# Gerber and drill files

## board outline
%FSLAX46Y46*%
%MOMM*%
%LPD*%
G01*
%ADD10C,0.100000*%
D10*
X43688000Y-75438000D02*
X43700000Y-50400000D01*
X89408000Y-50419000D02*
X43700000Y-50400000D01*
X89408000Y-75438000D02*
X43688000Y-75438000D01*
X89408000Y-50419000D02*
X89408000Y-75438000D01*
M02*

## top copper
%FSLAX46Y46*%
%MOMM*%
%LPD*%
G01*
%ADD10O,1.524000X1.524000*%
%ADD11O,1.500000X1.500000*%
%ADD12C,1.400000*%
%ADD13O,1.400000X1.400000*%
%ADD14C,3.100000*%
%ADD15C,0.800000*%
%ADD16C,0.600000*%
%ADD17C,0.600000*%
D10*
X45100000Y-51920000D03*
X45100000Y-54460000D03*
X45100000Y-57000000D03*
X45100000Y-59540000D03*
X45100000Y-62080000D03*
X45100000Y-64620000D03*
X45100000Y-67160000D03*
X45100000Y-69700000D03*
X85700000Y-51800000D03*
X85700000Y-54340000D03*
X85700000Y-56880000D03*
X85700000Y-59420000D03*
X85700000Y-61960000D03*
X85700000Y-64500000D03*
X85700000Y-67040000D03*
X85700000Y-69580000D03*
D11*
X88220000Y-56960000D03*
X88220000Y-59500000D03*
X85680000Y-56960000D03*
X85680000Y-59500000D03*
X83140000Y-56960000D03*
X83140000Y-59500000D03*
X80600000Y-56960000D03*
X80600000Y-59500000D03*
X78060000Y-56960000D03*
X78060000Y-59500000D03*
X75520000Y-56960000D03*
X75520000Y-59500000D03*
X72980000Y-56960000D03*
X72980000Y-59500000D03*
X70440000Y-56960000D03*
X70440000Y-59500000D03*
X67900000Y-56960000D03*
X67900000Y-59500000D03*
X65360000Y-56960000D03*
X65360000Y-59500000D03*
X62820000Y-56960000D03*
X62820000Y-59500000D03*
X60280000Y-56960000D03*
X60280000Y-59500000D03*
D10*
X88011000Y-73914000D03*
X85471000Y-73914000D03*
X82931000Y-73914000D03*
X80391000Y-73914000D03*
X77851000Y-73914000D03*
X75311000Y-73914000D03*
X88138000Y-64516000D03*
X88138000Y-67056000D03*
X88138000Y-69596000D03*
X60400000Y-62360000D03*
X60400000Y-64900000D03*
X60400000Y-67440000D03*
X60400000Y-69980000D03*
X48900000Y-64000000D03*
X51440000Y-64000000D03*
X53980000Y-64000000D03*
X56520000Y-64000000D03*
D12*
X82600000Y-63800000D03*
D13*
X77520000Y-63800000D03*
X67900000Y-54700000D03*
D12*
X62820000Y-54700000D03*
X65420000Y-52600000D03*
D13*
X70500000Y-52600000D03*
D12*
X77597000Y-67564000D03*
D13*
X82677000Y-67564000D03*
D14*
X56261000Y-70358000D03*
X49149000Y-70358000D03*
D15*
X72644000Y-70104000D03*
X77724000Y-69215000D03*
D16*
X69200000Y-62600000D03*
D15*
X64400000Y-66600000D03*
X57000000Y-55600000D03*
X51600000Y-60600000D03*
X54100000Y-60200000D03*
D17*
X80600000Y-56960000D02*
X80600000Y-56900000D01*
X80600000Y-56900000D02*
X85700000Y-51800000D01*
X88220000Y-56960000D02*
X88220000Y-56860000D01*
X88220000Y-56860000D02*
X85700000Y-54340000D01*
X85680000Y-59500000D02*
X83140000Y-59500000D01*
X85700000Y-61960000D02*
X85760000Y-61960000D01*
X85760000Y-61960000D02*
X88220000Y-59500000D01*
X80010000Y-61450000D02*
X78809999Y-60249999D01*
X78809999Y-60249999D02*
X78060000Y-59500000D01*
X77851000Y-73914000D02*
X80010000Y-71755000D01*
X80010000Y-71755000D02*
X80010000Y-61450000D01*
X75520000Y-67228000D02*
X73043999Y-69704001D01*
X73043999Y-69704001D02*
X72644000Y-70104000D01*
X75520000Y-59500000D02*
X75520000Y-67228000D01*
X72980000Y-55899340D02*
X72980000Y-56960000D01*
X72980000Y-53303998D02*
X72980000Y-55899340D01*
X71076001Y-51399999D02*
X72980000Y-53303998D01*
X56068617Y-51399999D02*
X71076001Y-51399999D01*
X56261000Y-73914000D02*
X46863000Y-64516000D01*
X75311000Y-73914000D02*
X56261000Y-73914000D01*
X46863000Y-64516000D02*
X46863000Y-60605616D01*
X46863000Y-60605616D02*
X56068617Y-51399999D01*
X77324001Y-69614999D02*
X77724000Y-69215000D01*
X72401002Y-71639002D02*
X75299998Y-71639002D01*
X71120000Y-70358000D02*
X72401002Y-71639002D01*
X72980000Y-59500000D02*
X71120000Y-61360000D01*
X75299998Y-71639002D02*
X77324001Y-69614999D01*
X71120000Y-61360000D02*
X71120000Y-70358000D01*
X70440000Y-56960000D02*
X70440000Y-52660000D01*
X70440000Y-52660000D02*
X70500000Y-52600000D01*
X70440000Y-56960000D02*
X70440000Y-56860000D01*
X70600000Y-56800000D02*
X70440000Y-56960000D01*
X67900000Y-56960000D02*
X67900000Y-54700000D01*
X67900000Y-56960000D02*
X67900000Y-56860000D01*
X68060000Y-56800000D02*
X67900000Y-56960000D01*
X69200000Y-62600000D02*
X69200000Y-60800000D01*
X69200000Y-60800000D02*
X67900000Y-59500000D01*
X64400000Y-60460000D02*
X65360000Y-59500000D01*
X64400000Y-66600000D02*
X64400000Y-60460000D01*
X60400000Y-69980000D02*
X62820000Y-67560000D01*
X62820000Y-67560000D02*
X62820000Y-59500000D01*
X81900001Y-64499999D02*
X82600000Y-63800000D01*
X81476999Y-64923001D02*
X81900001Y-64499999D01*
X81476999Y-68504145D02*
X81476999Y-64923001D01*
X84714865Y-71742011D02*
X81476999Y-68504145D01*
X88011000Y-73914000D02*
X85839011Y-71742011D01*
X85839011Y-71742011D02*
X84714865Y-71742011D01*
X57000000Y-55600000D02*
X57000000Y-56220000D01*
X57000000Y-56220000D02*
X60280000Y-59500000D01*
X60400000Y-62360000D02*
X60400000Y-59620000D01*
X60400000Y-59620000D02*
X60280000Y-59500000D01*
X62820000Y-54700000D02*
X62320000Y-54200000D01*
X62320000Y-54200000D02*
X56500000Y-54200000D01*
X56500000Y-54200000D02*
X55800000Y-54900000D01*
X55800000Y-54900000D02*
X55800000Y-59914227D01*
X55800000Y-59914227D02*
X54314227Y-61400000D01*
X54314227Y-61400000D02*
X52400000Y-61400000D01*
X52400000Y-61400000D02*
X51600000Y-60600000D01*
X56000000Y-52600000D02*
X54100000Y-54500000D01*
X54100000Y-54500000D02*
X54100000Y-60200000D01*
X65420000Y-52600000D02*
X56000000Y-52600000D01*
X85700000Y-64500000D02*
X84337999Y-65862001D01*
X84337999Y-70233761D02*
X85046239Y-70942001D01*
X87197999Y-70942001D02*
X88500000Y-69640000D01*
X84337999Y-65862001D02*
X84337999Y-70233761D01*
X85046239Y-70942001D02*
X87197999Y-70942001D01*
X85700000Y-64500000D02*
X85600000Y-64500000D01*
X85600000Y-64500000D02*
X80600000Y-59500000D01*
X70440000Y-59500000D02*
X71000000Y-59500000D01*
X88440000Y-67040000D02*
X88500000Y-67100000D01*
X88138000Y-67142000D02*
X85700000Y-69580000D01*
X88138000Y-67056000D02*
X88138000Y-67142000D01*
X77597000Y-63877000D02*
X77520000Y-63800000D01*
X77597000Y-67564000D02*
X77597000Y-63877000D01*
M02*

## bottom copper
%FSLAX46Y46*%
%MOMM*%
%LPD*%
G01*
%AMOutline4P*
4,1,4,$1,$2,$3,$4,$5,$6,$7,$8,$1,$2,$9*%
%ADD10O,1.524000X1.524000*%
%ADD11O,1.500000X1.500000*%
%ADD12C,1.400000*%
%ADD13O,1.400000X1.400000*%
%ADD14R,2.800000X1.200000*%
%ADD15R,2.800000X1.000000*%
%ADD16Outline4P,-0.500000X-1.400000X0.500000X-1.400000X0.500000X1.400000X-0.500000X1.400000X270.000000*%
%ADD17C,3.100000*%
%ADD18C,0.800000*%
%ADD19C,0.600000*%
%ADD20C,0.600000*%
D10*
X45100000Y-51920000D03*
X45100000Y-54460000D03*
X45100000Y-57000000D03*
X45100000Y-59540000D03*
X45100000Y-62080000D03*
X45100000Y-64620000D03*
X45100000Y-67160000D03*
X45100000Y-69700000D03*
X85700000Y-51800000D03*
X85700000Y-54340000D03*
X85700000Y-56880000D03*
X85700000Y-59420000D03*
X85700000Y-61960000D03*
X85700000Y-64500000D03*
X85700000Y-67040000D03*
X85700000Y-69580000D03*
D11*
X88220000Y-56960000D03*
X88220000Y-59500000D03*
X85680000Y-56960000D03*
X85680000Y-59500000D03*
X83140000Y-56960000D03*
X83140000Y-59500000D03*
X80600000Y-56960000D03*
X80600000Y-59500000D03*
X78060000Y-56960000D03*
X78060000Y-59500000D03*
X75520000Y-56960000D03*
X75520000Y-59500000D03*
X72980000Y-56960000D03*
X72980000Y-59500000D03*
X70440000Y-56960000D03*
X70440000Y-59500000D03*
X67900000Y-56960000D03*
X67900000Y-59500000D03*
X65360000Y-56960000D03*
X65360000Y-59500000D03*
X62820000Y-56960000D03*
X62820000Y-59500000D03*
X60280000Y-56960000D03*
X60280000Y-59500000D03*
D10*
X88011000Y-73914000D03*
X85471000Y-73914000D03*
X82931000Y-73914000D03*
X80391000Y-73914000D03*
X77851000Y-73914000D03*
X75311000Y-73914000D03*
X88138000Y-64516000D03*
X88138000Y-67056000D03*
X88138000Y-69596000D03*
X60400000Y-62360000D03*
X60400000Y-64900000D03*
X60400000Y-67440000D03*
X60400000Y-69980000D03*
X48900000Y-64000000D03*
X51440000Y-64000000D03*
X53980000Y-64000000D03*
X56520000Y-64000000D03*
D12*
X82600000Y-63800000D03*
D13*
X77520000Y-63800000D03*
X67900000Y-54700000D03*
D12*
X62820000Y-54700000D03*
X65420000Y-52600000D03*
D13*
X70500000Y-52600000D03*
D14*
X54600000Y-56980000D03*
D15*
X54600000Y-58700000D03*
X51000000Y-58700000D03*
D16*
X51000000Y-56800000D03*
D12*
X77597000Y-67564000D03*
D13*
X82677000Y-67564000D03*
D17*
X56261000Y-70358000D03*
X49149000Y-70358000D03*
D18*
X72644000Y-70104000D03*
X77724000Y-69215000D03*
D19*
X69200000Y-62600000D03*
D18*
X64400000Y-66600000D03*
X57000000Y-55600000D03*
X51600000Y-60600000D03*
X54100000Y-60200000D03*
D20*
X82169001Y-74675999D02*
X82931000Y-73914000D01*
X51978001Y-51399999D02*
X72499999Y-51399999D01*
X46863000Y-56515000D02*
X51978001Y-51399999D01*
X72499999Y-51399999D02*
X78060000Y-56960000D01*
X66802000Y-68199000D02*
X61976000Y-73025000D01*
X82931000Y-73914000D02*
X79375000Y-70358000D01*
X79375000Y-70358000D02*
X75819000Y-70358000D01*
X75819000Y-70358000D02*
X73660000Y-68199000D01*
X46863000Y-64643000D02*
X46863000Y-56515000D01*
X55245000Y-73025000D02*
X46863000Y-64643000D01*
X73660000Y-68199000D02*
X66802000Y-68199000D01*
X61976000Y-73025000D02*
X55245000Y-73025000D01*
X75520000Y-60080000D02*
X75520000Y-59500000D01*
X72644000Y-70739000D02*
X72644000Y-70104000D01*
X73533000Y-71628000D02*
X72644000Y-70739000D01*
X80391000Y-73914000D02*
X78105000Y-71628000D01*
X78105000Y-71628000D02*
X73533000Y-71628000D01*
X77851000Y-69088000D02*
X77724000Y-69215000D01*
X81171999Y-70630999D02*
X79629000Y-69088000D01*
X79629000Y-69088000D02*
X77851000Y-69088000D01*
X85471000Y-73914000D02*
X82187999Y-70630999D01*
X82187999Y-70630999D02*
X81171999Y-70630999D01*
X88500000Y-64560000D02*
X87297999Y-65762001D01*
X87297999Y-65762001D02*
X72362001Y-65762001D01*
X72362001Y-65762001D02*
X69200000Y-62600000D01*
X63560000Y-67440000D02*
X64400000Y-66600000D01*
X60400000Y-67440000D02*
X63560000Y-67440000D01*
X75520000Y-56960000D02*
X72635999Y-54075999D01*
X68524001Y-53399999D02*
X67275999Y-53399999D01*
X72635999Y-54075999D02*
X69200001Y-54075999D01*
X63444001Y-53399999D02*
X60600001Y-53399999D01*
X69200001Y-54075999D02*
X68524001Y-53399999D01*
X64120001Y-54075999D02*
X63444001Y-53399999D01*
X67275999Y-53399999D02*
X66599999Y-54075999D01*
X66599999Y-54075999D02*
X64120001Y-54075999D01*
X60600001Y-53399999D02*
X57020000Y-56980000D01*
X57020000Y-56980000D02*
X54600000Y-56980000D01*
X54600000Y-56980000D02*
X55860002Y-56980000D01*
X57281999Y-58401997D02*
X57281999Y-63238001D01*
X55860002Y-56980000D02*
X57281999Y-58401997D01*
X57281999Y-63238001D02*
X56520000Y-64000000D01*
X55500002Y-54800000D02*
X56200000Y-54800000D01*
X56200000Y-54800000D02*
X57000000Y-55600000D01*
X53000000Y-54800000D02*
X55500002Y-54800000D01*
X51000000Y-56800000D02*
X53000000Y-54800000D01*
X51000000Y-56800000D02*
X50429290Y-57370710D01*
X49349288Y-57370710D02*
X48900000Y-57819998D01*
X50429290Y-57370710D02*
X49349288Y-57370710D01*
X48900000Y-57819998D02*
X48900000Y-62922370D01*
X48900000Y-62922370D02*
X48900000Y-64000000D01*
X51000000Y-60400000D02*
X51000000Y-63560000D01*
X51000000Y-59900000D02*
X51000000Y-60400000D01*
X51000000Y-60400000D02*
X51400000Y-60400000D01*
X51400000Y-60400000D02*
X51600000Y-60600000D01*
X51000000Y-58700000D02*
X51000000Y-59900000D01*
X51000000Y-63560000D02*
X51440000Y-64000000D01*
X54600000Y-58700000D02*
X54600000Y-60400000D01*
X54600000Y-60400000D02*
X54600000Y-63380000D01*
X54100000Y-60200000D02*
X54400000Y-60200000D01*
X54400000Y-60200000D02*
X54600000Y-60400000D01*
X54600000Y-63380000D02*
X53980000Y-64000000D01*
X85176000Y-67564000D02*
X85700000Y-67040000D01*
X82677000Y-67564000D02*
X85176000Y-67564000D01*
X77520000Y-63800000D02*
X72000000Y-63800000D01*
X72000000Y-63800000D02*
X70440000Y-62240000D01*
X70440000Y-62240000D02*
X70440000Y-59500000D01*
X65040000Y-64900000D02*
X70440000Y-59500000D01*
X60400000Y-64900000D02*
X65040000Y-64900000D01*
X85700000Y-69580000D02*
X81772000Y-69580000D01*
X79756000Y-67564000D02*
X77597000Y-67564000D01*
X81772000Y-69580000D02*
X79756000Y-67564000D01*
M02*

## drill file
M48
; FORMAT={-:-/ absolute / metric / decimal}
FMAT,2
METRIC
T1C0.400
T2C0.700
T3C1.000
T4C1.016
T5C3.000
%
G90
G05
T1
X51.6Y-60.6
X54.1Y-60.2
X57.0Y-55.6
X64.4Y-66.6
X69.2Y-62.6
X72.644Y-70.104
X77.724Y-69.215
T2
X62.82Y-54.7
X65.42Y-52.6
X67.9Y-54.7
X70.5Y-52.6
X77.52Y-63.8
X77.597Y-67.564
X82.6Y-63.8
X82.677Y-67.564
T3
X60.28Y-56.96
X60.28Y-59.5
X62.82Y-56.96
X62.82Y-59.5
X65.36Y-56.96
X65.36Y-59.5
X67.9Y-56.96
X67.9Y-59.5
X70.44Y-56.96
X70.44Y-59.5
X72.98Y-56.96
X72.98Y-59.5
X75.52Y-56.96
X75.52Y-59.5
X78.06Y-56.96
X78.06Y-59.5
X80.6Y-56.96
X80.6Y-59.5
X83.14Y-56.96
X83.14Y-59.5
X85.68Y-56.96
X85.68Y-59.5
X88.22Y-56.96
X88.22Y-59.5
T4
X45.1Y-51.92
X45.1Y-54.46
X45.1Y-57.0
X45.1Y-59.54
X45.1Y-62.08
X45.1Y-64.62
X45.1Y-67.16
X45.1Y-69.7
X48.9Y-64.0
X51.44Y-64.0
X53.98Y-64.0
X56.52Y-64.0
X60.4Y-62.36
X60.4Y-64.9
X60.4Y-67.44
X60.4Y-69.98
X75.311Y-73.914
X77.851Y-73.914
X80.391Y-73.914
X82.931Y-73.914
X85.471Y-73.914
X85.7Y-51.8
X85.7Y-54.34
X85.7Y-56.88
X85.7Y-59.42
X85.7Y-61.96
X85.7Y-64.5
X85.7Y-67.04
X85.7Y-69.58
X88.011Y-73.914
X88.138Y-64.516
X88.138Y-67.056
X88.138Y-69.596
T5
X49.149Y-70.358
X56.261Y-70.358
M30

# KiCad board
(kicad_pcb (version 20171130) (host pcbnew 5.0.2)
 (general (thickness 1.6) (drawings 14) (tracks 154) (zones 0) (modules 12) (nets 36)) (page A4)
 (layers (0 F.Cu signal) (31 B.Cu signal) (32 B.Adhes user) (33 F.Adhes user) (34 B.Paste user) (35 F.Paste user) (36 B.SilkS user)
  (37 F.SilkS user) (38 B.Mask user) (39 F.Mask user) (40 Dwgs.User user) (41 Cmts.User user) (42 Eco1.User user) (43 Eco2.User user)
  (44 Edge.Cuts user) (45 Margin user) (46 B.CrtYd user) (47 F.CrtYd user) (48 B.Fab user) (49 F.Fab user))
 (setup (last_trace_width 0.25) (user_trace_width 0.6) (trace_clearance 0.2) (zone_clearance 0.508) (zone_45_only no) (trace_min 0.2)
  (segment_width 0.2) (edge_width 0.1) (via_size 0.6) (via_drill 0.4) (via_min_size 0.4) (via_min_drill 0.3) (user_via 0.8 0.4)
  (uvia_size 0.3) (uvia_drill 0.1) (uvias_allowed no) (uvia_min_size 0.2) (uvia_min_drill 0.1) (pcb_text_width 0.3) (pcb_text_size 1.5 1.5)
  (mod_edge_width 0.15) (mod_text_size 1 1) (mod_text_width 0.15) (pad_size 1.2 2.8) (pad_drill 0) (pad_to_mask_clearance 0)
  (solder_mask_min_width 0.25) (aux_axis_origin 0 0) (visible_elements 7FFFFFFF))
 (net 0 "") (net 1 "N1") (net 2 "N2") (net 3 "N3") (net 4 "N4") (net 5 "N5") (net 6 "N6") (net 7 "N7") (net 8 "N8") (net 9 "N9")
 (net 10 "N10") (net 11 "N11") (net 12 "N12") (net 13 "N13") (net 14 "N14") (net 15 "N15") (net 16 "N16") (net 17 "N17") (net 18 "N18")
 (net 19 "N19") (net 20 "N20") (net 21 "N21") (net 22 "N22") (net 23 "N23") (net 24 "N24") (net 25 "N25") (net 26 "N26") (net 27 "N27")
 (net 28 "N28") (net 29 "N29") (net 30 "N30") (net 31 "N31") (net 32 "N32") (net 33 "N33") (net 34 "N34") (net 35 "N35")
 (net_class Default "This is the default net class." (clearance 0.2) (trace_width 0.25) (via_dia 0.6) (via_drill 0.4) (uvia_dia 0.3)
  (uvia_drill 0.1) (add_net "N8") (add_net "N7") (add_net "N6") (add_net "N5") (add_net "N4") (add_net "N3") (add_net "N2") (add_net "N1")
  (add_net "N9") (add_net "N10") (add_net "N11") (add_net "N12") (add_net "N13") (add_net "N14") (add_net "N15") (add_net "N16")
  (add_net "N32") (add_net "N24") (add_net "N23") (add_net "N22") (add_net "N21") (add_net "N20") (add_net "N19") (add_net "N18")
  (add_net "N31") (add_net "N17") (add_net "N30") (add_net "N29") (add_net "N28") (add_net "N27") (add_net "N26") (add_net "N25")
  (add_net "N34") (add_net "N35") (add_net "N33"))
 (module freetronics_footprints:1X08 (layer F.Cu) (at 45.1 69.7 90)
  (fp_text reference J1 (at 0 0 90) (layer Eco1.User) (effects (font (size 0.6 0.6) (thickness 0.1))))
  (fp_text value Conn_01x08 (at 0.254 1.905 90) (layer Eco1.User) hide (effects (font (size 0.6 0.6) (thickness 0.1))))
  (pad 8 thru_hole oval (at 17.78 0 180) (size 1.524 1.524) (drill 1.016) (layers *.Cu *.Mask) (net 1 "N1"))
  (pad 7 thru_hole oval (at 15.24 0 180) (size 1.524 1.524) (drill 1.016) (layers *.Cu *.Mask) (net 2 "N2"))
  (pad 6 thru_hole oval (at 12.7 0 180) (size 1.524 1.524) (drill 1.016) (layers *.Cu *.Mask) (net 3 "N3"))
  (pad 5 thru_hole oval (at 10.16 0 180) (size 1.524 1.524) (drill 1.016) (layers *.Cu *.Mask) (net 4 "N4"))
  (pad 4 thru_hole oval (at 7.62 0 180) (size 1.524 1.524) (drill 1.016) (layers *.Cu *.Mask) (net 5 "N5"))
  (pad 3 thru_hole oval (at 5.08 0 180) (size 1.524 1.524) (drill 1.016) (layers *.Cu *.Mask) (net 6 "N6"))
  (pad 2 thru_hole oval (at 2.54 0 180) (size 1.524 1.524) (drill 1.016) (layers *.Cu *.Mask) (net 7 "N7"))
  (pad 1 thru_hole oval (at 0 0 180) (size 1.524 1.524) (drill 1.016) (layers *.Cu *.Mask) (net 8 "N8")))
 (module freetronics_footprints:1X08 (layer F.Cu) (at 85.7 51.8 270)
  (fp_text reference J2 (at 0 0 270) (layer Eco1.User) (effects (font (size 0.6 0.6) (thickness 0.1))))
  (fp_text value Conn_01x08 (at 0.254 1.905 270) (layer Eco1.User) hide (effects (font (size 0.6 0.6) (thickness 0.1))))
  (pad 1 thru_hole oval (at 0 0) (size 1.524 1.524) (drill 1.016) (layers *.Cu *.Mask) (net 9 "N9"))
  (pad 2 thru_hole oval (at 2.54 0) (size 1.524 1.524) (drill 1.016) (layers *.Cu *.Mask) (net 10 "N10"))
  (pad 3 thru_hole oval (at 5.08 0) (size 1.524 1.524) (drill 1.016) (layers *.Cu *.Mask) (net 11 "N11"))
  (pad 4 thru_hole oval (at 7.62 0) (size 1.524 1.524) (drill 1.016) (layers *.Cu *.Mask) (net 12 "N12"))
  (pad 5 thru_hole oval (at 10.16 0) (size 1.524 1.524) (drill 1.016) (layers *.Cu *.Mask) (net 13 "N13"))
  (pad 6 thru_hole oval (at 12.7 0) (size 1.524 1.524) (drill 1.016) (layers *.Cu *.Mask) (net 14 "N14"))
  (pad 7 thru_hole oval (at 15.24 0) (size 1.524 1.524) (drill 1.016) (layers *.Cu *.Mask) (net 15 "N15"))
  (pad 8 thru_hole oval (at 17.78 0) (size 1.524 1.524) (drill 1.016) (layers *.Cu *.Mask) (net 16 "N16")))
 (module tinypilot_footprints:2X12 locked (layer F.Cu) (at 60.28 59.5)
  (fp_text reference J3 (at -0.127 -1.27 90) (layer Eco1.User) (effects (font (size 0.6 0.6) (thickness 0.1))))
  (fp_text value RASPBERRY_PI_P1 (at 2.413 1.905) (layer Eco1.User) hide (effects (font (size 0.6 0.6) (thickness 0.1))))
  (pad 24 thru_hole oval (at 27.94 -2.54) (size 1.5 1.5) (drill 1) (layers *.Cu *.Mask) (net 10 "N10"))
  (pad 23 thru_hole oval (at 27.94 0) (size 1.5 1.5) (drill 1) (layers *.Cu *.Mask) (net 13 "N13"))
  (pad 22 thru_hole oval (at 25.4 -2.54) (size 1.5 1.5) (drill 1) (layers *.Cu *.Mask) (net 11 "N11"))
  (pad 21 thru_hole oval (at 25.4 0) (size 1.5 1.5) (drill 1) (layers *.Cu *.Mask) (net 12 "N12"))
  (pad 20 thru_hole oval (at 22.86 -2.54) (size 1.5 1.5) (drill 1) (layers *.Cu *.Mask) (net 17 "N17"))
  (pad 19 thru_hole oval (at 22.86 0) (size 1.5 1.5) (drill 1) (layers *.Cu *.Mask) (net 12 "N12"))
  (pad 18 thru_hole oval (at 20.32 -2.54) (size 1.5 1.5) (drill 1) (layers *.Cu *.Mask) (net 9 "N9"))
  (pad 17 thru_hole oval (at 20.32 0) (size 1.5 1.5) (drill 1) (layers *.Cu *.Mask) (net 14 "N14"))
  (pad 16 thru_hole oval (at 17.78 -2.54) (size 1.5 1.5) (drill 1) (layers *.Cu *.Mask) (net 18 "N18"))
  (pad 15 thru_hole oval (at 17.78 0) (size 1.5 1.5) (drill 1) (layers *.Cu *.Mask) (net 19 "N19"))
  (pad 14 thru_hole oval (at 15.24 -2.54) (size 1.5 1.5) (drill 1) (layers *.Cu *.Mask) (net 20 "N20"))
  (pad 13 thru_hole oval (at 15.24 0) (size 1.5 1.5) (drill 1) (layers *.Cu *.Mask) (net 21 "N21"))
  (pad 12 thru_hole oval (at 12.7 -2.54) (size 1.5 1.5) (drill 1) (layers *.Cu *.Mask) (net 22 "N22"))
  (pad 11 thru_hole oval (at 12.7 0) (size 1.5 1.5) (drill 1) (layers *.Cu *.Mask) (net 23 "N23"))
  (pad 10 thru_hole oval (at 10.16 -2.54) (size 1.5 1.5) (drill 1) (layers *.Cu *.Mask) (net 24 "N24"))
  (pad 9 thru_hole oval (at 10.16 0) (size 1.5 1.5) (drill 1) (layers *.Cu *.Mask) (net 16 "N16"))
  (pad 8 thru_hole oval (at 7.62 -2.54) (size 1.5 1.5) (drill 1) (layers *.Cu *.Mask) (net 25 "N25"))
  (pad 7 thru_hole oval (at 7.62 0) (size 1.5 1.5) (drill 1) (layers *.Cu *.Mask) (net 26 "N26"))
  (pad 6 thru_hole oval (at 5.08 -2.54) (size 1.5 1.5) (drill 1) (layers *.Cu *.Mask) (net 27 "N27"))
  (pad 5 thru_hole oval (at 5.08 0) (size 1.5 1.5) (drill 1) (layers *.Cu *.Mask) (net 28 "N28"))
  (pad 4 thru_hole oval (at 2.54 -2.54) (size 1.5 1.5) (drill 1) (layers *.Cu *.Mask) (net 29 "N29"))
  (pad 3 thru_hole oval (at 2.54 0) (size 1.5 1.5) (drill 1) (layers *.Cu *.Mask) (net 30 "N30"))
  (pad 2 thru_hole oval (at 0 -2.54) (size 1.5 1.5) (drill 1) (layers *.Cu *.Mask) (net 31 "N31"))
  (pad 1 thru_hole oval (at 0 0) (size 1.5 1.5) (drill 1) (layers *.Cu *.Mask) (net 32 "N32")))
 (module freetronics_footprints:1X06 (layer F.Cu) (at 88.011 73.914 180)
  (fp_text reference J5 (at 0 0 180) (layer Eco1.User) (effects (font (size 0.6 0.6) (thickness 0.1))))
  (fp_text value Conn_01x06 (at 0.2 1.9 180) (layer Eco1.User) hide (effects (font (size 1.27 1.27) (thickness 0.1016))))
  (pad 1 thru_hole oval (at 0 0 270) (size 1.524 1.524) (drill 1.016) (layers *.Cu *.Mask) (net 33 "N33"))
  (pad 2 thru_hole oval (at 2.54 0 270) (size 1.524 1.524) (drill 1.016) (layers *.Cu *.Mask) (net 23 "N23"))
  (pad 3 thru_hole oval (at 5.08 0 270) (size 1.524 1.524) (drill 1.016) (layers *.Cu *.Mask) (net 18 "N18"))
  (pad 4 thru_hole oval (at 7.62 0 270) (size 1.524 1.524) (drill 1.016) (layers *.Cu *.Mask) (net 21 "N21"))
  (pad 5 thru_hole oval (at 10.16 0 270) (size 1.524 1.524) (drill 1.016) (layers *.Cu *.Mask) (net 19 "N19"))
  (pad 6 thru_hole oval (at 12.7 0 270) (size 1.524 1.524) (drill 1.016) (layers *.Cu *.Mask) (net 22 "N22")))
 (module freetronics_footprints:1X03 (layer F.Cu) (at 88.138 64.516 270)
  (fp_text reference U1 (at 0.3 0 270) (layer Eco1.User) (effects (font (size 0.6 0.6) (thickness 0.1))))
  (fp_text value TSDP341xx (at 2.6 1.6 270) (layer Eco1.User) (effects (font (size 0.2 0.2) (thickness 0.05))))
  (pad 1 thru_hole oval (at 0 0) (size 1.524 1.524) (drill 1.016) (layers *.Cu *.Mask) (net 26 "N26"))
  (pad 2 thru_hole oval (at 2.54 0) (size 1.524 1.524) (drill 1.016) (layers *.Cu *.Mask) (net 16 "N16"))
  (pad 3 thru_hole oval (at 5.08 0) (size 1.524 1.524) (drill 1.016) (layers *.Cu *.Mask) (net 14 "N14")))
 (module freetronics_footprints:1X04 (layer F.Cu) (at 60.4 62.36 270)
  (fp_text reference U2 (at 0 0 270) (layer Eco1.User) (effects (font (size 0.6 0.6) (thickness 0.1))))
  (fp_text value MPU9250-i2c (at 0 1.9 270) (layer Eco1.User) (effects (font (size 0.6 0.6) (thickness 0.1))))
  (pad 1 thru_hole oval (at 0 0) (size 1.524 1.524) (drill 1.016) (layers *.Cu *.Mask) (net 32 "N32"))
  (pad 2 thru_hole oval (at 2.54 0) (size 1.524 1.524) (drill 1.016) (layers *.Cu *.Mask) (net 16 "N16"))
  (pad 3 thru_hole oval (at 5.08 0) (size 1.524 1.524) (drill 1.016) (layers *.Cu *.Mask) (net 28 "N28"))
  (pad 4 thru_hole oval (at 7.62 0) (size 1.524 1.524) (drill 1.016) (layers *.Cu *.Mask) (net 30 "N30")))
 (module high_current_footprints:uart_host (layer F.Cu) (at 48.9 64)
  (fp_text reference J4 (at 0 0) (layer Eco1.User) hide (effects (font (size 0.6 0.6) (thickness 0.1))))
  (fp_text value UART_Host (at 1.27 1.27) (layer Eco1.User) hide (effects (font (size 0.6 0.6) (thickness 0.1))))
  (pad 1 thru_hole oval (at 0 0 90) (size 1.524 1.524) (drill 1.016) (layers *.Cu *.Mask) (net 32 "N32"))
  (pad 2 thru_hole oval (at 2.54 0 90) (size 1.524 1.524) (drill 1.016) (layers *.Cu *.Mask) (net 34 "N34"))
  (pad 3 thru_hole oval (at 5.08 0 90) (size 1.524 1.524) (drill 1.016) (layers *.Cu *.Mask) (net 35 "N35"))
  (pad 4 thru_hole oval (at 7.62 0 90) (size 1.524 1.524) (drill 1.016) (layers *.Cu *.Mask) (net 20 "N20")))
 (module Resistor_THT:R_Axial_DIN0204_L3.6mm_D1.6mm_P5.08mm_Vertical (layer B.Cu) (at 82.6 63.8 180)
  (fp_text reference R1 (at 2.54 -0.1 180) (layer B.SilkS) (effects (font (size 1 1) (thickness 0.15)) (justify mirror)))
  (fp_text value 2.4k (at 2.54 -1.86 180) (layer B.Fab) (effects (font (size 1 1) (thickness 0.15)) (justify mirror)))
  (pad 1 thru_hole circle (at 0 0 180) (size 1.4 1.4) (drill 0.7) (layers *.Cu *.Mask) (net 33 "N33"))
  (pad 2 thru_hole oval (at 5.08 0 180) (size 1.4 1.4) (drill 0.7) (layers *.Cu *.Mask) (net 16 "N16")))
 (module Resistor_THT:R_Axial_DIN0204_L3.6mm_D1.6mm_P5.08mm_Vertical (layer B.Cu) (at 62.82 54.7)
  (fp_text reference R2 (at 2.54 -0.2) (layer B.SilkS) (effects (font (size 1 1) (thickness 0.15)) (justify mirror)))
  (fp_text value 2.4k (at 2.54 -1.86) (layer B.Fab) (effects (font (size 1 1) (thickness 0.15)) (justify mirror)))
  (pad 2 thru_hole oval (at 5.08 0) (size 1.4 1.4) (drill 0.7) (layers *.Cu *.Mask) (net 25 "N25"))
  (pad 1 thru_hole circle (at 0 0) (size 1.4 1.4) (drill 0.7) (layers *.Cu *.Mask) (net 34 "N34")))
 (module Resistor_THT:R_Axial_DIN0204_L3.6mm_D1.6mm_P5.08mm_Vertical (layer B.Cu) (at 65.42 52.6)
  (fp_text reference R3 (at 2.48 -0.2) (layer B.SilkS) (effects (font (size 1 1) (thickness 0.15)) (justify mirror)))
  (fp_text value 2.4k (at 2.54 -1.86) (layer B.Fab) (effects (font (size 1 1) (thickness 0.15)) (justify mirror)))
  (pad 1 thru_hole circle (at 0 0) (size 1.4 1.4) (drill 0.7) (layers *.Cu *.Mask) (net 35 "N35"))
  (pad 2 thru_hole oval (at 5.08 0) (size 1.4 1.4) (drill 0.7) (layers *.Cu *.Mask) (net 24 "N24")))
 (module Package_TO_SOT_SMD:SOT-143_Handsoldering (layer B.Cu) (at 52.8 57.75 180)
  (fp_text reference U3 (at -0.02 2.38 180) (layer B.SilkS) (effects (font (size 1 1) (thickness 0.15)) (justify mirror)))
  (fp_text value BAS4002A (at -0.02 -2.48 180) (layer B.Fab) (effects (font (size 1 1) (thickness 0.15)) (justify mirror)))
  (pad 1 smd rect (at -1.8 0.77 270) (size 1.2 2.8) (layers B.Cu B.Paste B.Mask) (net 20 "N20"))
  (pad 2 smd rect (at -1.8 -0.95 270) (size 1 2.8) (layers B.Cu B.Paste B.Mask) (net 35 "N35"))
  (pad 3 smd rect (at 1.8 -0.95 270) (size 1 2.8) (layers B.Cu B.Paste B.Mask) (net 34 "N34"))
  (pad 4 smd trapezoid (at 1.8 0.95 270) (size 1 2.8) (layers B.Cu B.Paste B.Mask) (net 32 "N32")))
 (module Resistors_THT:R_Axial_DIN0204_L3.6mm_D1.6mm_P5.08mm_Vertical (layer B.Cu) (at 77.597 67.564)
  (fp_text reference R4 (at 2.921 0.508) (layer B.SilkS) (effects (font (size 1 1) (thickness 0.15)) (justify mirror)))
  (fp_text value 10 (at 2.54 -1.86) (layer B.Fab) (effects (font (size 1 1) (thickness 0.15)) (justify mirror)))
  (pad 1 thru_hole circle (at 0 0) (size 1.4 1.4) (drill 0.7) (layers *.Cu *.Mask) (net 16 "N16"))
  (pad 2 thru_hole oval (at 5.08 0) (size 1.4 1.4) (drill 0.7) (layers *.Cu *.Mask) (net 15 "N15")))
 (gr_line (start 43.688 75.438) (end 43.7 50.4) (layer Edge.Cuts) (width 0.1))
 (gr_line (start 89.408 50.419) (end 43.7 50.4) (layer Edge.Cuts) (width 0.1))
 (gr_line (start 89.408 75.438) (end 43.688 75.438) (layer Edge.Cuts) (width 0.1))
 (gr_line (start 89.408 50.419) (end 89.408 75.438) (layer Edge.Cuts) (width 0.1))
 (via (at 56.261 70.358) (size 3.1) (drill 3) (layers F.Cu B.Cu) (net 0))
 (via (at 49.149 70.358) (size 3.1) (drill 3) (layers F.Cu B.Cu) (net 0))
 (segment (start 80.6 56.96) (end 80.6 56.9) (width 0.6) (layer F.Cu) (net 9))
 (segment (start 80.6 56.9) (end 85.7 51.8) (width 0.6) (layer F.Cu) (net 9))
 (segment (start 88.22 56.96) (end 88.22 56.86) (width 0.6) (layer F.Cu) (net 10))
 (segment (start 88.22 56.86) (end 85.7 54.34) (width 0.6) (layer F.Cu) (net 10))
 (segment (start 85.68 59.5) (end 83.14 59.5) (width 0.6) (layer F.Cu) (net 12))
 (segment (start 85.7 61.96) (end 85.76 61.96) (width 0.6) (layer F.Cu) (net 13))
 (segment (start 85.76 61.96) (end 88.22 59.5) (width 0.6) (layer F.Cu) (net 13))
 (segment (start 82.169001 74.675999) (end 82.931 73.914) (width 0.6) (layer B.Cu) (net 18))
 (segment (start 51.978001 51.399999) (end 72.499999 51.399999) (width 0.6) (layer B.Cu) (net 18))
 (segment (start 46.863 56.515) (end 51.978001 51.399999) (width 0.6) (layer B.Cu) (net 18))
 (segment (start 72.499999 51.399999) (end 78.06 56.96) (width 0.6) (layer B.Cu) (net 18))
 (segment (start 66.802 68.199) (end 61.976 73.025) (width 0.6) (layer B.Cu) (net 18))
 (segment (start 82.931 73.914) (end 79.375 70.358) (width 0.6) (layer B.Cu) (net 18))
 (segment (start 79.375 70.358) (end 75.819 70.358) (width 0.6) (layer B.Cu) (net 18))
 (segment (start 75.819 70.358) (end 73.66 68.199) (width 0.6) (layer B.Cu) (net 18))
 (segment (start 46.863 64.643) (end 46.863 56.515) (width 0.6) (layer B.Cu) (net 18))
 (segment (start 55.245 73.025) (end 46.863 64.643) (width 0.6) (layer B.Cu) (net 18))
 (segment (start 73.66 68.199) (end 66.802 68.199) (width 0.6) (layer B.Cu) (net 18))
 (segment (start 61.976 73.025) (end 55.245 73.025) (width 0.6) (layer B.Cu) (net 18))
 (segment (start 80.01 61.45) (end 78.809999 60.249999) (width 0.6) (layer F.Cu) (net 19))
 (segment (start 78.809999 60.249999) (end 78.06 59.5) (width 0.6) (layer F.Cu) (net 19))
 (segment (start 77.851 73.914) (end 80.01 71.755) (width 0.6) (layer F.Cu) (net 19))
 (segment (start 80.01 71.755) (end 80.01 61.45) (width 0.6) (layer F.Cu) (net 19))
 (segment (start 75.52 60.08) (end 75.52 59.5) (width 0.6) (layer B.Cu) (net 21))
 (via (at 72.644 70.104) (size 0.8) (drill 0.4) (layers F.Cu B.Cu) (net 21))
 (segment (start 75.52 67.228) (end 73.043999 69.704001) (width 0.6) (layer F.Cu) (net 21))
 (segment (start 73.043999 69.704001) (end 72.644 70.104) (width 0.6) (layer F.Cu) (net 21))
 (segment (start 75.52 59.5) (end 75.52 67.228) (width 0.6) (layer F.Cu) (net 21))
 (segment (start 72.644 70.739) (end 72.644 70.104) (width 0.6) (layer B.Cu) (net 21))
 (segment (start 73.533 71.628) (end 72.644 70.739) (width 0.6) (layer B.Cu) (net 21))
 (segment (start 80.391 73.914) (end 78.105 71.628) (width 0.6) (layer B.Cu) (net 21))
 (segment (start 78.105 71.628) (end 73.533 71.628) (width 0.6) (layer B.Cu) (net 21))
 (segment (start 72.98 55.89934) (end 72.98 56.96) (width 0.6) (layer F.Cu) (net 22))
 (segment (start 72.98 53.303998) (end 72.98 55.89934) (width 0.6) (layer F.Cu) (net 22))
 (segment (start 71.076001 51.399999) (end 72.98 53.303998) (width 0.6) (layer F.Cu) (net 22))
 (segment (start 56.068617 51.399999) (end 71.076001 51.399999) (width 0.6) (layer F.Cu) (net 22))
 (segment (start 56.261 73.914) (end 46.863 64.516) (width 0.6) (layer F.Cu) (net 22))
 (segment (start 75.311 73.914) (end 56.261 73.914) (width 0.6) (layer F.Cu) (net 22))
 (segment (start 46.863 64.516) (end 46.863 60.605616) (width 0.6) (layer F.Cu) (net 22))
 (segment (start 46.863 60.605616) (end 56.068617 51.399999) (width 0.6) (layer F.Cu) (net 22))
 (via (at 77.724 69.215) (size 0.8) (drill 0.4) (layers F.Cu B.Cu) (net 23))
 (segment (start 77.851 69.088) (end 77.724 69.215) (width 0.6) (layer B.Cu) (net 23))
 (segment (start 81.171999 70.630999) (end 79.629 69.088) (width 0.6) (layer B.Cu) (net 23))
 (segment (start 79.629 69.088) (end 77.851 69.088) (width 0.6) (layer B.Cu) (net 23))
 (segment (start 85.471 73.914) (end 82.187999 70.630999) (width 0.6) (layer B.Cu) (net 23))
 (segment (start 82.187999 70.630999) (end 81.171999 70.630999) (width 0.6) (layer B.Cu) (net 23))
 (segment (start 77.324001 69.614999) (end 77.724 69.215) (width 0.6) (layer F.Cu) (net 23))
 (segment (start 72.401002 71.639002) (end 75.299998 71.639002) (width 0.6) (layer F.Cu) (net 23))
 (segment (start 71.12 70.358) (end 72.401002 71.639002) (width 0.6) (layer F.Cu) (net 23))
 (segment (start 72.98 59.5) (end 71.12 61.36) (width 0.6) (layer F.Cu) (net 23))
 (segment (start 75.299998 71.639002) (end 77.324001 69.614999) (width 0.6) (layer F.Cu) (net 23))
 (segment (start 71.12 61.36) (end 71.12 70.358) (width 0.6) (layer F.Cu) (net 23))
 (segment (start 70.44 56.96) (end 70.44 52.66) (width 0.6) (layer F.Cu) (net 24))
 (segment (start 70.44 52.66) (end 70.5 52.6) (width 0.6) (layer F.Cu) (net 24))
 (segment (start 70.44 56.96) (end 70.44 56.86) (width 0.6) (layer F.Cu) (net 24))
 (segment (start 70.6 56.8) (end 70.44 56.96) (width 0.6) (layer F.Cu) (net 24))
 (segment (start 67.9 56.96) (end 67.9 54.7) (width 0.6) (layer F.Cu) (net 25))
 (segment (start 67.9 56.96) (end 67.9 56.86) (width 0.6) (layer F.Cu) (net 25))
 (segment (start 68.06 56.8) (end 67.9 56.96) (width 0.6) (layer F.Cu) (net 25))
 (segment (start 69.2 62.6) (end 69.2 60.8) (width 0.6) (layer F.Cu) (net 26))
 (segment (start 69.2 60.8) (end 67.9 59.5) (width 0.6) (layer F.Cu) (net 26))
 (segment (start 88.5 64.56) (end 87.297999 65.762001) (width 0.6) (layer B.Cu) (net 26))
 (segment (start 87.297999 65.762001) (end 72.362001 65.762001) (width 0.6) (layer B.Cu) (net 26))
 (segment (start 72.362001 65.762001) (end 69.2 62.6) (width 0.6) (layer B.Cu) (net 26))
 (via (at 69.2 62.6) (size 0.6) (drill 0.4) (layers F.Cu B.Cu) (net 26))
 (segment (start 63.56 67.44) (end 64.4 66.6) (width 0.6) (layer B.Cu) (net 28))
 (segment (start 64.4 60.46) (end 65.36 59.5) (width 0.6) (layer F.Cu) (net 28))
 (segment (start 64.4 66.6) (end 64.4 60.46) (width 0.6) (layer F.Cu) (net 28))
 (segment (start 60.4 67.44) (end 63.56 67.44) (width 0.6) (layer B.Cu) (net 28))
 (via (at 64.4 66.6) (size 0.8) (drill 0.4) (layers F.Cu B.Cu) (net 28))
 (segment (start 60.4 69.98) (end 62.82 67.56) (width 0.6) (layer F.Cu) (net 30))
 (segment (start 62.82 67.56) (end 62.82 59.5) (width 0.6) (layer F.Cu) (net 30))
 (segment (start 81.900001 64.499999) (end 82.6 63.8) (width 0.6) (layer F.Cu) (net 33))
 (segment (start 81.476999 64.923001) (end 81.900001 64.499999) (width 0.6) (layer F.Cu) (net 33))
 (segment (start 81.476999 68.504145) (end 81.476999 64.923001) (width 0.6) (layer F.Cu) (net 33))
 (segment (start 84.714865 71.742011) (end 81.476999 68.504145) (width 0.6) (layer F.Cu) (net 33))
 (segment (start 88.011 73.914) (end 85.839011 71.742011) (width 0.6) (layer F.Cu) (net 33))
 (segment (start 85.839011 71.742011) (end 84.714865 71.742011) (width 0.6) (layer F.Cu) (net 33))
 (segment (start 75.52 56.96) (end 72.635999 54.075999) (width 0.6) (layer B.Cu) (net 20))
 (segment (start 68.524001 53.399999) (end 67.275999 53.399999) (width 0.6) (layer B.Cu) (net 20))
 (segment (start 72.635999 54.075999) (end 69.200001 54.075999) (width 0.6) (layer B.Cu) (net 20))
 (segment (start 63.444001 53.399999) (end 60.600001 53.399999) (width 0.6) (layer B.Cu) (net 20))
 (segment (start 69.200001 54.075999) (end 68.524001 53.399999) (width 0.6) (layer B.Cu) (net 20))
 (segment (start 64.120001 54.075999) (end 63.444001 53.399999) (width 0.6) (layer B.Cu) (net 20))
 (segment (start 67.275999 53.399999) (end 66.599999 54.075999) (width 0.6) (layer B.Cu) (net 20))
 (segment (start 66.599999 54.075999) (end 64.120001 54.075999) (width 0.6) (layer B.Cu) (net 20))
 (segment (start 60.600001 53.399999) (end 57.02 56.98) (width 0.6) (layer B.Cu) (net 20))
 (segment (start 57.02 56.98) (end 54.6 56.98) (width 0.6) (layer B.Cu) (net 20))
 (segment (start 54.6 56.98) (end 55.860002 56.98) (width 0.6) (layer B.Cu) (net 20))
 (segment (start 57.281999 58.401997) (end 57.281999 63.238001) (width 0.6) (layer B.Cu) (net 20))
 (segment (start 55.860002 56.98) (end 57.281999 58.401997) (width 0.6) (layer B.Cu) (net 20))
 (segment (start 57.281999 63.238001) (end 56.52 64) (width 0.6) (layer B.Cu) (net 20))
 (segment (start 57 55.6) (end 57 56.22) (width 0.6) (layer F.Cu) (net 32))
 (segment (start 57 56.22) (end 60.28 59.5) (width 0.6) (layer F.Cu) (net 32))
 (segment (start 55.500002 54.8) (end 56.2 54.8) (width 0.6) (layer B.Cu) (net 32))
 (segment (start 56.2 54.8) (end 57 55.6) (width 0.6) (layer B.Cu) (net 32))
 (via (at 57 55.6) (size 0.8) (drill 0.4) (layers F.Cu B.Cu) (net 32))
 (segment (start 53 54.8) (end 55.500002 54.8) (width 0.6) (layer B.Cu) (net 32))
 (segment (start 51 56.8) (end 53 54.8) (width 0.6) (layer B.Cu) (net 32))
 (segment (start 51 56.8) (end 50.42929 57.37071) (width 0.6) (layer B.Cu) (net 32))
 (segment (start 49.349288 57.37071) (end 48.9 57.819998) (width 0.6) (layer B.Cu) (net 32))
 (segment (start 50.42929 57.37071) (end 49.349288 57.37071) (width 0.6) (layer B.Cu) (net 32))
 (segment (start 48.9 57.819998) (end 48.9 62.92237) (width 0.6) (layer B.Cu) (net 32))
 (segment (start 48.9 62.92237) (end 48.9 64) (width 0.6) (layer B.Cu) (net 32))
 (segment (start 60.4 62.36) (end 60.4 59.62) (width 0.6) (layer F.Cu) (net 32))
 (segment (start 60.4 59.62) (end 60.28 59.5) (width 0.6) (layer F.Cu) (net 32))
 (segment (start 62.82 54.7) (end 62.32 54.2) (width 0.6) (layer F.Cu) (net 34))
 (segment (start 62.32 54.2) (end 56.5 54.2) (width 0.6) (layer F.Cu) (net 34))
 (segment (start 56.5 54.2) (end 55.8 54.9) (width 0.6) (layer F.Cu) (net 34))
 (segment (start 55.8 54.9) (end 55.8 59.914227) (width 0.6) (layer F.Cu) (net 34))
 (segment (start 55.8 59.914227) (end 54.314227 61.4) (width 0.6) (layer F.Cu) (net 34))
 (segment (start 54.314227 61.4) (end 52.4 61.4) (width 0.6) (layer F.Cu) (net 34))
 (segment (start 52.4 61.4) (end 51.6 60.6) (width 0.6) (layer F.Cu) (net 34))
 (segment (start 51 60.4) (end 51 63.56) (width 0.6) (layer B.Cu) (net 34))
 (segment (start 51 59.9) (end 51 60.4) (width 0.6) (layer B.Cu) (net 34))
 (segment (start 51 60.4) (end 51.4 60.4) (width 0.6) (layer B.Cu) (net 34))
 (segment (start 51.4 60.4) (end 51.6 60.6) (width 0.6) (layer B.Cu) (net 34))
 (via (at 51.6 60.6) (size 0.8) (drill 0.4) (layers F.Cu B.Cu) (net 34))
 (segment (start 51 58.7) (end 51 59.9) (width 0.6) (layer B.Cu) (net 34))
 (segment (start 51 63.56) (end 51.44 64) (width 0.6) (layer B.Cu) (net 34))
 (segment (start 54.6 58.7) (end 54.6 60.4) (width 0.6) (layer B.Cu) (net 35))
 (segment (start 54.6 60.4) (end 54.6 63.38) (width 0.6) (layer B.Cu) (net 35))
 (segment (start 54.1 60.2) (end 54.4 60.2) (width 0.6) (layer B.Cu) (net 35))
 (segment (start 54.4 60.2) (end 54.6 60.4) (width 0.6) (layer B.Cu) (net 35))
 (segment (start 56 52.6) (end 54.1 54.5) (width 0.6) (layer F.Cu) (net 35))
 (segment (start 54.1 54.5) (end 54.1 60.2) (width 0.6) (layer F.Cu) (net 35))
 (via (at 54.1 60.2) (size 0.8) (drill 0.4) (layers F.Cu B.Cu) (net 35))
 (segment (start 65.42 52.6) (end 56 52.6) (width 0.6) (layer F.Cu) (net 35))
 (segment (start 54.6 63.38) (end 53.98 64) (width 0.6) (layer B.Cu) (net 35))
 (segment (start 85.7 64.5) (end 84.337999 65.862001) (width 0.6) (layer F.Cu) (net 14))
 (segment (start 84.337999 70.233761) (end 85.046239 70.942001) (width 0.6) (layer F.Cu) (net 14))
 (segment (start 87.197999 70.942001) (end 88.5 69.64) (width 0.6) (layer F.Cu) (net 14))
 (segment (start 84.337999 65.862001) (end 84.337999 70.233761) (width 0.6) (layer F.Cu) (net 14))
 (segment (start 85.046239 70.942001) (end 87.197999 70.942001) (width 0.6) (layer F.Cu) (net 14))
 (segment (start 85.7 64.5) (end 85.6 64.5) (width 0.6) (layer F.Cu) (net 14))
 (segment (start 85.6 64.5) (end 80.6 59.5) (width 0.6) (layer F.Cu) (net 14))
 (segment (start 85.176 67.564) (end 85.7 67.04) (width 0.6) (layer B.Cu) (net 15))
 (segment (start 82.677 67.564) (end 85.176 67.564) (width 0.6) (layer B.Cu) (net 15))
 (segment (start 77.52 63.8) (end 72 63.8) (width 0.6) (layer B.Cu) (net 16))
 (segment (start 72 63.8) (end 70.44 62.24) (width 0.6) (layer B.Cu) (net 16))
 (segment (start 70.44 62.24) (end 70.44 59.5) (width 0.6) (layer B.Cu) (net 16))
 (segment (start 70.44 59.5) (end 71 59.5) (width 0.6) (layer F.Cu) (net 16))
 (segment (start 65.04 64.9) (end 70.44 59.5) (width 0.6) (layer B.Cu) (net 16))
 (segment (start 60.4 64.9) (end 65.04 64.9) (width 0.6) (layer B.Cu) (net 16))
 (segment (start 88.44 67.04) (end 88.5 67.1) (width 0.6) (layer F.Cu) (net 16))
 (segment (start 88.138 67.142) (end 85.7 69.58) (width 0.6) (layer F.Cu) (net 16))
 (segment (start 88.138 67.056) (end 88.138 67.142) (width 0.6) (layer F.Cu) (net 16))
 (segment (start 77.597 63.877) (end 77.52 63.8) (width 0.6) (layer F.Cu) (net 16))
 (segment (start 77.597 67.564) (end 77.597 63.877) (width 0.6) (layer F.Cu) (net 16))
 (segment (start 85.7 69.58) (end 81.772 69.58) (width 0.6) (layer B.Cu) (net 16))
 (segment (start 79.756 67.564) (end 77.597 67.564) (width 0.6) (layer B.Cu) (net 16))
 (segment (start 81.772 69.58) (end 79.756 67.564) (width 0.6) (layer B.Cu) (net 16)))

